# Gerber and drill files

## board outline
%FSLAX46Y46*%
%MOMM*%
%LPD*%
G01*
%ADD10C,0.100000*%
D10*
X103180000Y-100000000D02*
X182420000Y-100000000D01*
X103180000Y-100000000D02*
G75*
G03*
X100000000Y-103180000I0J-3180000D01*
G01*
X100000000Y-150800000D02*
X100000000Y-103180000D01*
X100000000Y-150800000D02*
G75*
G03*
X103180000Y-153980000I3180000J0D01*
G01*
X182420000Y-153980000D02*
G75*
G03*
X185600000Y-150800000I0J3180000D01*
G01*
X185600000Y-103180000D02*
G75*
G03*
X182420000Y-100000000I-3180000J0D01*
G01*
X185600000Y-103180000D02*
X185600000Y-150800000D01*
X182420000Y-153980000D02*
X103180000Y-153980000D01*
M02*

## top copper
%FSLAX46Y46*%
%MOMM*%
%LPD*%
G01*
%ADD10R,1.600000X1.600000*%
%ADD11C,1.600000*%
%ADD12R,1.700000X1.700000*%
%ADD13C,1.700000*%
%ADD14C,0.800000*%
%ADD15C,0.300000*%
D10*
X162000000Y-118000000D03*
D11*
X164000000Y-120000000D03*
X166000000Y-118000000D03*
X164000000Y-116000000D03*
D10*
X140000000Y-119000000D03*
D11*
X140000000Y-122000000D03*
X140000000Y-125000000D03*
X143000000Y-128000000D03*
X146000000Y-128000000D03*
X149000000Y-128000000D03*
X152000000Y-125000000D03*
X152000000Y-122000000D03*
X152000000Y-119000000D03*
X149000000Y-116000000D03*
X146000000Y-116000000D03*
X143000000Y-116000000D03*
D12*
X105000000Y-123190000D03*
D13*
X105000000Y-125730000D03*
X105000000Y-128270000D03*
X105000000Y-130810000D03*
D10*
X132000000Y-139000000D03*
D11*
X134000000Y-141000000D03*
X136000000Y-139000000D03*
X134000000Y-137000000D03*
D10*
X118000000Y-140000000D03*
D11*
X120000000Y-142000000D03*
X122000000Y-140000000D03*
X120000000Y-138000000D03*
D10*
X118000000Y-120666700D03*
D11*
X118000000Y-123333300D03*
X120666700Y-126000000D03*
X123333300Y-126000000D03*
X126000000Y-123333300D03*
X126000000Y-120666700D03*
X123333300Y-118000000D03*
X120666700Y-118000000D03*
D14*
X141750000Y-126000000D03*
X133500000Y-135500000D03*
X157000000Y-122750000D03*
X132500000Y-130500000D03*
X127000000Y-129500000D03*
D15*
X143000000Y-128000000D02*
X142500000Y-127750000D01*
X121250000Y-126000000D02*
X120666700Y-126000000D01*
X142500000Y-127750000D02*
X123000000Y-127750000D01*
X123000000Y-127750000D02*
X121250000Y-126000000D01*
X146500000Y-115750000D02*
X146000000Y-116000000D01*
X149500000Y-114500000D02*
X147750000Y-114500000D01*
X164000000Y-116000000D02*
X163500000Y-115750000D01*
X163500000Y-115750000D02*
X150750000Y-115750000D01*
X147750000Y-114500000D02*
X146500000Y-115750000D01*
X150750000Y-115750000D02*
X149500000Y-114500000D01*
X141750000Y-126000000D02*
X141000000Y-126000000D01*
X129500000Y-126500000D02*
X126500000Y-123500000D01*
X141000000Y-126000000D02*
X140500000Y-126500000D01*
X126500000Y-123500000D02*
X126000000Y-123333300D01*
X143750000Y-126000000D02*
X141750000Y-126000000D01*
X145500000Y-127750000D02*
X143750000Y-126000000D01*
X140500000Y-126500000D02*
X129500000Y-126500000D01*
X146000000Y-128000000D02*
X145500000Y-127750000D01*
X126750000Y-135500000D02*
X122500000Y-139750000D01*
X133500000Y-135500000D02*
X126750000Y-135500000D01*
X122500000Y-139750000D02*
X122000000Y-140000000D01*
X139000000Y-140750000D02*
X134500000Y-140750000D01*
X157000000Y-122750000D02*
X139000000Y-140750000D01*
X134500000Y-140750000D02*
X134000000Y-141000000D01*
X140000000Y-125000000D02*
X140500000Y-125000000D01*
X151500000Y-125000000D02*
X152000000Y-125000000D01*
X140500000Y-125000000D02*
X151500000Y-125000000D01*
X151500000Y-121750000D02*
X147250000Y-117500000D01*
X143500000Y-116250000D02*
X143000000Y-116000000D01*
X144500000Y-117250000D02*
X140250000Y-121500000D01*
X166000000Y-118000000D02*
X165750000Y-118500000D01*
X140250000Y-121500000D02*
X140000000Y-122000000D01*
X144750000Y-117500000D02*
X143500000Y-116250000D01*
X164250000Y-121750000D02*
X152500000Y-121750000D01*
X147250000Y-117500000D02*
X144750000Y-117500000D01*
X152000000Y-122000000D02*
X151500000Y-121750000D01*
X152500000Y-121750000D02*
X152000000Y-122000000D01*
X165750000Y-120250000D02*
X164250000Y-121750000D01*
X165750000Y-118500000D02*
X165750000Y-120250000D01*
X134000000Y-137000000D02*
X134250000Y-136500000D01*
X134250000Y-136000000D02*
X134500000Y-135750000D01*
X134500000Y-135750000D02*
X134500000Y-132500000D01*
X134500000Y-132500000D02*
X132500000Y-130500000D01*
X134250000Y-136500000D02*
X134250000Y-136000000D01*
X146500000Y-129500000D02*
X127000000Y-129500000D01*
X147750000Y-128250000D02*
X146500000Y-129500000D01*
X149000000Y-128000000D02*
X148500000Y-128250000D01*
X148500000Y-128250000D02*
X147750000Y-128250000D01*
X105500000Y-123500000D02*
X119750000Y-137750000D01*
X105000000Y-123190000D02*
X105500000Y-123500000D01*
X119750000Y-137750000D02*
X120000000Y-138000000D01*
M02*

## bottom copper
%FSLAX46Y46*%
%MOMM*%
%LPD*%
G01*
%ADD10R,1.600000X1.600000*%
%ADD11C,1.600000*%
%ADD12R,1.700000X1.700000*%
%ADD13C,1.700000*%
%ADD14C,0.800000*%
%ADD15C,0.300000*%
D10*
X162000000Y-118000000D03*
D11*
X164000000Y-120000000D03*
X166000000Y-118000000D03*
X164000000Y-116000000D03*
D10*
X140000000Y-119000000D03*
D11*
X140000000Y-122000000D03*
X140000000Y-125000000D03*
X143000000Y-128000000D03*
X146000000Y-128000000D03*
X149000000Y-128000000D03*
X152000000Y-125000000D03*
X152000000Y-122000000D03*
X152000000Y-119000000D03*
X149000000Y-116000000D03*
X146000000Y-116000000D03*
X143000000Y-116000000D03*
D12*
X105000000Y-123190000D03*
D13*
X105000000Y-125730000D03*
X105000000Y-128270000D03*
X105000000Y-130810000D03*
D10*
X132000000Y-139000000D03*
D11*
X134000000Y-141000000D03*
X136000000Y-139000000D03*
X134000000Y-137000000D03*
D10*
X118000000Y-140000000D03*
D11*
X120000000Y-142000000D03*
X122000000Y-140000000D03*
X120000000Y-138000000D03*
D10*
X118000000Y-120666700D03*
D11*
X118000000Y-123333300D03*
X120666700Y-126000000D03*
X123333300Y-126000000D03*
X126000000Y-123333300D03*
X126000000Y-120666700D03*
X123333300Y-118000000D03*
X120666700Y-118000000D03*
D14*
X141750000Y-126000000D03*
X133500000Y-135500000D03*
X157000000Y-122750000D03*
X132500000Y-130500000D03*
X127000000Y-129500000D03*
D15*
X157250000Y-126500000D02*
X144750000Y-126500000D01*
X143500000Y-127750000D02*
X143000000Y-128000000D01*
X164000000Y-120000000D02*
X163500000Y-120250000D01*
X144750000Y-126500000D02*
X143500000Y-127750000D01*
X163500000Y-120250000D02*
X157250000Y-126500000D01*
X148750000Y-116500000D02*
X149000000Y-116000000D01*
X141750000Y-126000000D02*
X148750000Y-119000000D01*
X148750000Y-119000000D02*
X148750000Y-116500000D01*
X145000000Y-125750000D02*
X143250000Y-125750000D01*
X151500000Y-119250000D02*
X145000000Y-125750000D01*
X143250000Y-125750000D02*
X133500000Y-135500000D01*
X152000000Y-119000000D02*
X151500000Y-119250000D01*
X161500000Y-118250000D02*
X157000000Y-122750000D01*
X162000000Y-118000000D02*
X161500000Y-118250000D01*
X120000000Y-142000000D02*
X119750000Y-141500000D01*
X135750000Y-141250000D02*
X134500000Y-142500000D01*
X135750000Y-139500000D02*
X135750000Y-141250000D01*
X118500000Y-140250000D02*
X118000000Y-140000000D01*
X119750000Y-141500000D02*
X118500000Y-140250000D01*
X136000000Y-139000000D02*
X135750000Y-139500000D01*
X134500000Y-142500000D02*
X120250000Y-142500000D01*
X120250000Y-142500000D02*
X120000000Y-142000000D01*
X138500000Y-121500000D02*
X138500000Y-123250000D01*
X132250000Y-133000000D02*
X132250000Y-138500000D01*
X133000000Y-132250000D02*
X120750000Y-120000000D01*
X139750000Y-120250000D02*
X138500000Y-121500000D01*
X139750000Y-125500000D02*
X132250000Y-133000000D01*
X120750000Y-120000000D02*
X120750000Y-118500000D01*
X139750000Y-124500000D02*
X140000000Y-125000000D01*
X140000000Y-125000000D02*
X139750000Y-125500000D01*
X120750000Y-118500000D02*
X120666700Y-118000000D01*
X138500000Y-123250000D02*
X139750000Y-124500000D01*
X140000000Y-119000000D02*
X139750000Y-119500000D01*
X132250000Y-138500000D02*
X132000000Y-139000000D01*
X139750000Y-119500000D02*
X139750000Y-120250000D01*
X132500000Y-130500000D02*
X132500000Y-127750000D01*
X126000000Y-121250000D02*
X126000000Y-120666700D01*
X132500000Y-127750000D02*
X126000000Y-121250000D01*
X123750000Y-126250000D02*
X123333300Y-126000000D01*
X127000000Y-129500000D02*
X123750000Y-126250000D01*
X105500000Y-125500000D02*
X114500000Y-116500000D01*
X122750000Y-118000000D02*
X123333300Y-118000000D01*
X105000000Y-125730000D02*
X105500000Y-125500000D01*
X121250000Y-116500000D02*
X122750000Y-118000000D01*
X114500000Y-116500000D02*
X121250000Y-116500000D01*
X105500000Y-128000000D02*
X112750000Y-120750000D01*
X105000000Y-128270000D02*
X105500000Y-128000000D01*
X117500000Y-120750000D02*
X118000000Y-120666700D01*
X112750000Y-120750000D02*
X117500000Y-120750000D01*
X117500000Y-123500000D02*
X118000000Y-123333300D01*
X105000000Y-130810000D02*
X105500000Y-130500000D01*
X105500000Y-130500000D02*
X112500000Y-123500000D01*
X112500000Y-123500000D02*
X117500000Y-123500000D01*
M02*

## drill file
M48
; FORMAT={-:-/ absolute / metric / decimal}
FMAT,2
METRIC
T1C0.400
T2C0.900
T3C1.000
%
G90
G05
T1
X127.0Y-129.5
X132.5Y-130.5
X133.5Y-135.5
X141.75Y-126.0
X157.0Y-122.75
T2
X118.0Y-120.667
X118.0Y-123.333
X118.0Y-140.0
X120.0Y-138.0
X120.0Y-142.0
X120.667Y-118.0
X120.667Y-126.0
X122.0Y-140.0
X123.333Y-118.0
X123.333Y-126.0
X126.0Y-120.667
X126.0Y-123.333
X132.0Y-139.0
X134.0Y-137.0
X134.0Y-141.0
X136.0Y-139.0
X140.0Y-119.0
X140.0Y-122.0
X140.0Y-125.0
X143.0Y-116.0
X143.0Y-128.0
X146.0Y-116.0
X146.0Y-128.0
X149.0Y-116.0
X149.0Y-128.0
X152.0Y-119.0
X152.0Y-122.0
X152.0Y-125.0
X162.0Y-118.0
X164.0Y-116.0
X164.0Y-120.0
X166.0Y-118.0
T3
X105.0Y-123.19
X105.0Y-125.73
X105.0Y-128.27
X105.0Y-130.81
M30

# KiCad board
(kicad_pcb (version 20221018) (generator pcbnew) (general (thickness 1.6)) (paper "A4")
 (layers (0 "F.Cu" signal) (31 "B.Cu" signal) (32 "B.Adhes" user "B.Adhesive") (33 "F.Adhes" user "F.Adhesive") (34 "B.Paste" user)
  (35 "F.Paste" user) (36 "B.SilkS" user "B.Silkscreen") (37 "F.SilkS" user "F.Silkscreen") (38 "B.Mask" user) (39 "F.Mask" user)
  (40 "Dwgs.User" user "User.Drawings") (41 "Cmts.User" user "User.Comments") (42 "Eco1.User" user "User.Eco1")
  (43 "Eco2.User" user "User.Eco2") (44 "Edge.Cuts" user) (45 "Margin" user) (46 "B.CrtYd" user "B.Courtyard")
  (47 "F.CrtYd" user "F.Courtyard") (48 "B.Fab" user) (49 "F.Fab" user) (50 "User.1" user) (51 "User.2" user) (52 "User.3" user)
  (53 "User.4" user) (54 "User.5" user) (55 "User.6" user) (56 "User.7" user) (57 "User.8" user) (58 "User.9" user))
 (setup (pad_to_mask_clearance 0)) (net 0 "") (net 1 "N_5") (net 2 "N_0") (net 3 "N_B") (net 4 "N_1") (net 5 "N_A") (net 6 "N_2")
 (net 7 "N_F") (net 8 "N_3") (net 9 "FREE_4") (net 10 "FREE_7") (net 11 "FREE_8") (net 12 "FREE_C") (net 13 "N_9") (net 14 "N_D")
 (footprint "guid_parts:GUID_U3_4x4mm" (layer "F.Cu") (at 164 118)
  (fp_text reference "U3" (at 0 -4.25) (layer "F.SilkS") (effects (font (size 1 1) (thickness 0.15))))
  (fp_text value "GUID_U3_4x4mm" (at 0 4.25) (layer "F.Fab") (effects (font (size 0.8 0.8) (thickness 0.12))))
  (pad "1" thru_hole rect (at -2 0) (size 1.6 1.6) (drill 0.9) (layers "*.Cu" "*.Mask") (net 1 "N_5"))
  (pad "2" thru_hole circle (at 0 2) (size 1.6 1.6) (drill 0.9) (layers "*.Cu" "*.Mask") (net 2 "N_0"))
  (pad "3" thru_hole circle (at 2 0) (size 1.6 1.6) (drill 0.9) (layers "*.Cu" "*.Mask") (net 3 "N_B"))
  (pad "4" thru_hole circle (at 0 -2) (size 1.6 1.6) (drill 0.9) (layers "*.Cu" "*.Mask") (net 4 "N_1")))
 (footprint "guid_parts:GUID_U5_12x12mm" (layer "F.Cu") (at 146 122)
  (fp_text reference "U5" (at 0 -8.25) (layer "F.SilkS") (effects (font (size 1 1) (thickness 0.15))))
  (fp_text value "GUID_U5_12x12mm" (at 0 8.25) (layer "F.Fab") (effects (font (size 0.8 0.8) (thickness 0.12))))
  (pad "1" thru_hole rect (at -6 -3) (size 1.6 1.6) (drill 0.9) (layers "*.Cu" "*.Mask") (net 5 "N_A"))
  (pad "2" thru_hole circle (at -6 0) (size 1.6 1.6) (drill 0.9) (layers "*.Cu" "*.Mask") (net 3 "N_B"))
  (pad "3" thru_hole circle (at -6 3) (size 1.6 1.6) (drill 0.9) (layers "*.Cu" "*.Mask") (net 5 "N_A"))
  (pad "4" thru_hole circle (at -3 6) (size 1.6 1.6) (drill 0.9) (layers "*.Cu" "*.Mask") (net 2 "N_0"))
  (pad "5" thru_hole circle (at 0 6) (size 1.6 1.6) (drill 0.9) (layers "*.Cu" "*.Mask") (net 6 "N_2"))
  (pad "6" thru_hole circle (at 3 6) (size 1.6 1.6) (drill 0.9) (layers "*.Cu" "*.Mask") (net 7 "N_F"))
  (pad "7" thru_hole circle (at 6 3) (size 1.6 1.6) (drill 0.9) (layers "*.Cu" "*.Mask") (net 5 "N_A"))
  (pad "8" thru_hole circle (at 6 0) (size 1.6 1.6) (drill 0.9) (layers "*.Cu" "*.Mask") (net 3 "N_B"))
  (pad "9" thru_hole circle (at 6 -3) (size 1.6 1.6) (drill 0.9) (layers "*.Cu" "*.Mask") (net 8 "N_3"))
  (pad "10" thru_hole circle (at 3 -6) (size 1.6 1.6) (drill 0.9) (layers "*.Cu" "*.Mask") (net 6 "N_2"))
  (pad "11" thru_hole circle (at 0 -6) (size 1.6 1.6) (drill 0.9) (layers "*.Cu" "*.Mask") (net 4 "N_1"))
  (pad "12" thru_hole circle (at -3 -6) (size 1.6 1.6) (drill 0.9) (layers "*.Cu" "*.Mask") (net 3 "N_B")))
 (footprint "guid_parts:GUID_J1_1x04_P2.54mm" (layer "F.Cu") (at 105 127)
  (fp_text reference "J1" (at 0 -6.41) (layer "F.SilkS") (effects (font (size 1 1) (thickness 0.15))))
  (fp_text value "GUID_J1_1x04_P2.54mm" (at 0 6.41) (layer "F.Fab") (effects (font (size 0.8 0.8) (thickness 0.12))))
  (pad "1" thru_hole rect (at 0 -3.81) (size 1.7 1.7) (drill 1) (layers "*.Cu" "*.Mask") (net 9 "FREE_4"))
  (pad "2" thru_hole circle (at 0 -1.27) (size 1.7 1.7) (drill 1) (layers "*.Cu" "*.Mask") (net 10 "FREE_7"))
  (pad "3" thru_hole circle (at 0 1.27) (size 1.7 1.7) (drill 1) (layers "*.Cu" "*.Mask") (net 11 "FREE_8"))
  (pad "4" thru_hole circle (at 0 3.81) (size 1.7 1.7) (drill 1) (layers "*.Cu" "*.Mask") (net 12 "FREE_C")))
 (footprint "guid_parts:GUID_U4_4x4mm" (layer "F.Cu") (at 134 139)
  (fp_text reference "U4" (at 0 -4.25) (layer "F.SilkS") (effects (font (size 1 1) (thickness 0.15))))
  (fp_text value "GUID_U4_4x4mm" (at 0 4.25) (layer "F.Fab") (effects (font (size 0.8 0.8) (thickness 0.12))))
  (pad "1" thru_hole rect (at -2 0) (size 1.6 1.6) (drill 0.9) (layers "*.Cu" "*.Mask") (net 5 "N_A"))
  (pad "2" thru_hole circle (at 0 2) (size 1.6 1.6) (drill 0.9) (layers "*.Cu" "*.Mask") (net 1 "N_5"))
  (pad "3" thru_hole circle (at 2 0) (size 1.6 1.6) (drill 0.9) (layers "*.Cu" "*.Mask") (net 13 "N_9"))
  (pad "4" thru_hole circle (at 0 -2) (size 1.6 1.6) (drill 0.9) (layers "*.Cu" "*.Mask") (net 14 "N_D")))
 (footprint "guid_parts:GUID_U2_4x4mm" (layer "F.Cu") (at 120 140)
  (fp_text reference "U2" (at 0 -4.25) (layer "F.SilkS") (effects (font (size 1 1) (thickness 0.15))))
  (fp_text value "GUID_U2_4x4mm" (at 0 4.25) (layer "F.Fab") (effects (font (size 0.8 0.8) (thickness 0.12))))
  (pad "1" thru_hole rect (at -2 0) (size 1.6 1.6) (drill 0.9) (layers "*.Cu" "*.Mask") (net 13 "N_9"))
  (pad "2" thru_hole circle (at 0 2) (size 1.6 1.6) (drill 0.9) (layers "*.Cu" "*.Mask") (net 13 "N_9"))
  (pad "3" thru_hole circle (at 2 0) (size 1.6 1.6) (drill 0.9) (layers "*.Cu" "*.Mask") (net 8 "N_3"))
  (pad "4" thru_hole circle (at 0 -2) (size 1.6 1.6) (drill 0.9) (layers "*.Cu" "*.Mask") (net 9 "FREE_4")))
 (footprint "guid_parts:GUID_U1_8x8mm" (layer "F.Cu") (at 122 122)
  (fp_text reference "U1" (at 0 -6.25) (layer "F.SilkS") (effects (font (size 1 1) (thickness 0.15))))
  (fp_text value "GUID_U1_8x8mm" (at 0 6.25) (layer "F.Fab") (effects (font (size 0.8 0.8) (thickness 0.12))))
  (pad "1" thru_hole rect (at -4 -1.3333) (size 1.6 1.6) (drill 0.9) (layers "*.Cu" "*.Mask") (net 11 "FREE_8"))
  (pad "2" thru_hole circle (at -4 1.3333) (size 1.6 1.6) (drill 0.9) (layers "*.Cu" "*.Mask") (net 12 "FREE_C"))
  (pad "3" thru_hole circle (at -1.3333 4) (size 1.6 1.6) (drill 0.9) (layers "*.Cu" "*.Mask") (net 2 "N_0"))
  (pad "4" thru_hole circle (at 1.3333 4) (size 1.6 1.6) (drill 0.9) (layers "*.Cu" "*.Mask") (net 7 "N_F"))
  (pad "5" thru_hole circle (at 4 1.3333) (size 1.6 1.6) (drill 0.9) (layers "*.Cu" "*.Mask") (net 6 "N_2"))
  (pad "6" thru_hole circle (at 4 -1.3333) (size 1.6 1.6) (drill 0.9) (layers "*.Cu" "*.Mask") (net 14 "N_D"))
  (pad "7" thru_hole circle (at 1.3333 -4) (size 1.6 1.6) (drill 0.9) (layers "*.Cu" "*.Mask") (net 10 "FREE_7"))
  (pad "8" thru_hole circle (at -1.3333 -4) (size 1.6 1.6) (drill 0.9) (layers "*.Cu" "*.Mask") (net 5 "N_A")))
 (gr_line (start 103.18 100) (end 182.42 100) (stroke (width 0.1) (type default)) (layer "Edge.Cuts"))
 (gr_arc (start 100 103.18) (mid 100.9314 100.9314) (end 103.18 100) (stroke (width 0.1) (type default)) (layer "Edge.Cuts"))
 (gr_line (start 100 150.8) (end 100 103.18) (stroke (width 0.1) (type default)) (layer "Edge.Cuts"))
 (gr_arc (start 103.18 153.98) (mid 100.9314 153.048599) (end 100 150.8) (stroke (width 0.1) (type default)) (layer "Edge.Cuts"))
 (gr_arc (start 185.6 150.8) (mid 184.668599 153.048599) (end 182.42 153.98) (stroke (width 0.1) (type default)) (layer "Edge.Cuts"))
 (gr_arc (start 182.42 100) (mid 184.668599 100.9314) (end 185.6 103.18) (stroke (width 0.1) (type default)) (layer "Edge.Cuts"))
 (gr_line (start 185.6 103.18) (end 185.6 150.8) (stroke (width 0.1) (type default)) (layer "Edge.Cuts"))
 (gr_line (start 182.42 153.98) (end 103.18 153.98) (stroke (width 0.1) (type default)) (layer "Edge.Cuts"))
 (segment (start 143 128) (end 142.5 127.75) (width 0.3) (layer "F.Cu") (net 2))
 (segment (start 121.25 126) (end 120.6667 126) (width 0.3) (layer "F.Cu") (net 2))
 (segment (start 142.5 127.75) (end 123 127.75) (width 0.3) (layer "F.Cu") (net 2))
 (segment (start 123 127.75) (end 121.25 126) (width 0.3) (layer "F.Cu") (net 2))
 (segment (start 157.25 126.5) (end 144.75 126.5) (width 0.3) (layer "B.Cu") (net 2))
 (segment (start 143.5 127.75) (end 143 128) (width 0.3) (layer "B.Cu") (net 2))
 (segment (start 164 120) (end 163.5 120.25) (width 0.3) (layer "B.Cu") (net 2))
 (segment (start 144.75 126.5) (end 143.5 127.75) (width 0.3) (layer "B.Cu") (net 2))
 (segment (start 163.5 120.25) (end 157.25 126.5) (width 0.3) (layer "B.Cu") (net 2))
 (segment (start 146.5 115.75) (end 146 116) (width 0.3) (layer "F.Cu") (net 4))
 (segment (start 149.5 114.5) (end 147.75 114.5) (width 0.3) (layer "F.Cu") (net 4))
 (segment (start 164 116) (end 163.5 115.75) (width 0.3) (layer "F.Cu") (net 4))
 (segment (start 163.5 115.75) (end 150.75 115.75) (width 0.3) (layer "F.Cu") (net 4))
 (segment (start 147.75 114.5) (end 146.5 115.75) (width 0.3) (layer "F.Cu") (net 4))
 (segment (start 150.75 115.75) (end 149.5 114.5) (width 0.3) (layer "F.Cu") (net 4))
 (segment (start 141.75 126) (end 141 126) (width 0.3) (layer "F.Cu") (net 6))
 (segment (start 129.5 126.5) (end 126.5 123.5) (width 0.3) (layer "F.Cu") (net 6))
 (segment (start 141 126) (end 140.5 126.5) (width 0.3) (layer "F.Cu") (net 6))
 (segment (start 126.5 123.5) (end 126 123.3333) (width 0.3) (layer "F.Cu") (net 6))
 (segment (start 143.75 126) (end 141.75 126) (width 0.3) (layer "F.Cu") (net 6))
 (segment (start 145.5 127.75) (end 143.75 126) (width 0.3) (layer "F.Cu") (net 6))
 (segment (start 140.5 126.5) (end 129.5 126.5) (width 0.3) (layer "F.Cu") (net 6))
 (segment (start 146 128) (end 145.5 127.75) (width 0.3) (layer "F.Cu") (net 6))
 (via (at 141.75 126) (size 0.8) (drill 0.4) (layers "F.Cu" "B.Cu") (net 6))
 (segment (start 148.75 116.5) (end 149 116) (width 0.3) (layer "B.Cu") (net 6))
 (segment (start 141.75 126) (end 148.75 119) (width 0.3) (layer "B.Cu") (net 6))
 (segment (start 148.75 119) (end 148.75 116.5) (width 0.3) (layer "B.Cu") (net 6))
 (segment (start 126.75 135.5) (end 122.5 139.75) (width 0.3) (layer "F.Cu") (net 8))
 (segment (start 133.5 135.5) (end 126.75 135.5) (width 0.3) (layer "F.Cu") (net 8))
 (segment (start 122.5 139.75) (end 122 140) (width 0.3) (layer "F.Cu") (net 8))
 (via (at 133.5 135.5) (size 0.8) (drill 0.4) (layers "F.Cu" "B.Cu") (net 8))
 (segment (start 145 125.75) (end 143.25 125.75) (width 0.3) (layer "B.Cu") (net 8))
 (segment (start 151.5 119.25) (end 145 125.75) (width 0.3) (layer "B.Cu") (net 8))
 (segment (start 143.25 125.75) (end 133.5 135.5) (width 0.3) (layer "B.Cu") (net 8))
 (segment (start 152 119) (end 151.5 119.25) (width 0.3) (layer "B.Cu") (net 8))
 (segment (start 139 140.75) (end 134.5 140.75) (width 0.3) (layer "F.Cu") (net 1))
 (segment (start 157 122.75) (end 139 140.75) (width 0.3) (layer "F.Cu") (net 1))
 (segment (start 134.5 140.75) (end 134 141) (width 0.3) (layer "F.Cu") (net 1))
 (via (at 157 122.75) (size 0.8) (drill 0.4) (layers "F.Cu" "B.Cu") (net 1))
 (segment (start 161.5 118.25) (end 157 122.75) (width 0.3) (layer "B.Cu") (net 1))
 (segment (start 162 118) (end 161.5 118.25) (width 0.3) (layer "B.Cu") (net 1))
 (segment (start 120 142) (end 119.75 141.5) (width 0.3) (layer "B.Cu") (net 13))
 (segment (start 135.75 141.25) (end 134.5 142.5) (width 0.3) (layer "B.Cu") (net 13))
 (segment (start 135.75 139.5) (end 135.75 141.25) (width 0.3) (layer "B.Cu") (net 13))
 (segment (start 118.5 140.25) (end 118 140) (width 0.3) (layer "B.Cu") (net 13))
 (segment (start 119.75 141.5) (end 118.5 140.25) (width 0.3) (layer "B.Cu") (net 13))
 (segment (start 136 139) (end 135.75 139.5) (width 0.3) (layer "B.Cu") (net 13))
 (segment (start 134.5 142.5) (end 120.25 142.5) (width 0.3) (layer "B.Cu") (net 13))
 (segment (start 120.25 142.5) (end 120 142) (width 0.3) (layer "B.Cu") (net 13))
 (segment (start 140 125) (end 140.5 125) (width 0.3) (layer "F.Cu") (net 5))
 (segment (start 151.5 125) (end 152 125) (width 0.3) (layer "F.Cu") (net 5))
 (segment (start 140.5 125) (end 151.5 125) (width 0.3) (layer "F.Cu") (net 5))
 (segment (start 138.5 121.5) (end 138.5 123.25) (width 0.3) (layer "B.Cu") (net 5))
 (segment (start 132.25 133) (end 132.25 138.5) (width 0.3) (layer "B.Cu") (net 5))
 (segment (start 133 132.25) (end 120.75 120) (width 0.3) (layer "B.Cu") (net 5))
 (segment (start 139.75 120.25) (end 138.5 121.5) (width 0.3) (layer "B.Cu") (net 5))
 (segment (start 139.75 125.5) (end 132.25 133) (width 0.3) (layer "B.Cu") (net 5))
 (segment (start 120.75 120) (end 120.75 118.5) (width 0.3) (layer "B.Cu") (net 5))
 (segment (start 139.75 124.5) (end 140 125) (width 0.3) (layer "B.Cu") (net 5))
 (segment (start 140 125) (end 139.75 125.5) (width 0.3) (layer "B.Cu") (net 5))
 (segment (start 120.75 118.5) (end 120.6667 118) (width 0.3) (layer "B.Cu") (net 5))
 (segment (start 138.5 123.25) (end 139.75 124.5) (width 0.3) (layer "B.Cu") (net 5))
 (segment (start 140 119) (end 139.75 119.5) (width 0.3) (layer "B.Cu") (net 5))
 (segment (start 132.25 138.5) (end 132 139) (width 0.3) (layer "B.Cu") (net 5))
 (segment (start 139.75 119.5) (end 139.75 120.25) (width 0.3) (layer "B.Cu") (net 5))
 (segment (start 151.5 121.75) (end 147.25 117.5) (width 0.3) (layer "F.Cu") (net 3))
 (segment (start 143.5 116.25) (end 143 116) (width 0.3) (layer "F.Cu") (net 3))
 (segment (start 144.5 117.25) (end 140.25 121.5) (width 0.3) (layer "F.Cu") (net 3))
 (segment (start 166 118) (end 165.75 118.5) (width 0.3) (layer "F.Cu") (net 3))
 (segment (start 140.25 121.5) (end 140 122) (width 0.3) (layer "F.Cu") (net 3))
 (segment (start 144.75 117.5) (end 143.5 116.25) (width 0.3) (layer "F.Cu") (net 3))
 (segment (start 164.25 121.75) (end 152.5 121.75) (width 0.3) (layer "F.Cu") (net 3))
 (segment (start 147.25 117.5) (end 144.75 117.5) (width 0.3) (layer "F.Cu") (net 3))
 (segment (start 152 122) (end 151.5 121.75) (width 0.3) (layer "F.Cu") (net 3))
 (segment (start 152.5 121.75) (end 152 122) (width 0.3) (layer "F.Cu") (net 3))
 (segment (start 165.75 120.25) (end 164.25 121.75) (width 0.3) (layer "F.Cu") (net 3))
 (segment (start 165.75 118.5) (end 165.75 120.25) (width 0.3) (layer "F.Cu") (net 3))
 (segment (start 134 137) (end 134.25 136.5) (width 0.3) (layer "F.Cu") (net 14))
 (segment (start 134.25 136) (end 134.5 135.75) (width 0.3) (layer "F.Cu") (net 14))
 (segment (start 134.5 135.75) (end 134.5 132.5) (width 0.3) (layer "F.Cu") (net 14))
 (segment (start 134.5 132.5) (end 132.5 130.5) (width 0.3) (layer "F.Cu") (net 14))
 (segment (start 134.25 136.5) (end 134.25 136) (width 0.3) (layer "F.Cu") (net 14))
 (via (at 132.5 130.5) (size 0.8) (drill 0.4) (layers "F.Cu" "B.Cu") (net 14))
 (segment (start 132.5 130.5) (end 132.5 127.75) (width 0.3) (layer "B.Cu") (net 14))
 (segment (start 126 121.25) (end 126 120.6667) (width 0.3) (layer "B.Cu") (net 14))
 (segment (start 132.5 127.75) (end 126 121.25) (width 0.3) (layer "B.Cu") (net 14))
 (segment (start 146.5 129.5) (end 127 129.5) (width 0.3) (layer "F.Cu") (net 7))
 (segment (start 147.75 128.25) (end 146.5 129.5) (width 0.3) (layer "F.Cu") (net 7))
 (segment (start 149 128) (end 148.5 128.25) (width 0.3) (layer "F.Cu") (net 7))
 (segment (start 148.5 128.25) (end 147.75 128.25) (width 0.3) (layer "F.Cu") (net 7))
 (via (at 127 129.5) (size 0.8) (drill 0.4) (layers "F.Cu" "B.Cu") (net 7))
 (segment (start 123.75 126.25) (end 123.3333 126) (width 0.3) (layer "B.Cu") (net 7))
 (segment (start 127 129.5) (end 123.75 126.25) (width 0.3) (layer "B.Cu") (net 7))
 (segment (start 105.5 123.5) (end 119.75 137.75) (width 0.3) (layer "F.Cu") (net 9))
 (segment (start 105 123.19) (end 105.5 123.5) (width 0.3) (layer "F.Cu") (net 9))
 (segment (start 119.75 137.75) (end 120 138) (width 0.3) (layer "F.Cu") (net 9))
 (segment (start 105.5 125.5) (end 114.5 116.5) (width 0.3) (layer "B.Cu") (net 10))
 (segment (start 122.75 118) (end 123.3333 118) (width 0.3) (layer "B.Cu") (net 10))
 (segment (start 105 125.73) (end 105.5 125.5) (width 0.3) (layer "B.Cu") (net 10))
 (segment (start 121.25 116.5) (end 122.75 118) (width 0.3) (layer "B.Cu") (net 10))
 (segment (start 114.5 116.5) (end 121.25 116.5) (width 0.3) (layer "B.Cu") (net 10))
 (segment (start 105.5 128) (end 112.75 120.75) (width 0.3) (layer "B.Cu") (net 11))
 (segment (start 105 128.27) (end 105.5 128) (width 0.3) (layer "B.Cu") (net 11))
 (segment (start 117.5 120.75) (end 118 120.6667) (width 0.3) (layer "B.Cu") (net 11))
 (segment (start 112.75 120.75) (end 117.5 120.75) (width 0.3) (layer "B.Cu") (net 11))
 (segment (start 117.5 123.5) (end 118 123.3333) (width 0.3) (layer "B.Cu") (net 12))
 (segment (start 105 130.81) (end 105.5 130.5) (width 0.3) (layer "B.Cu") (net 12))
 (segment (start 105.5 130.5) (end 112.5 123.5) (width 0.3) (layer "B.Cu") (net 12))
 (segment (start 112.5 123.5) (end 117.5 123.5) (width 0.3) (layer "B.Cu") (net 12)))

